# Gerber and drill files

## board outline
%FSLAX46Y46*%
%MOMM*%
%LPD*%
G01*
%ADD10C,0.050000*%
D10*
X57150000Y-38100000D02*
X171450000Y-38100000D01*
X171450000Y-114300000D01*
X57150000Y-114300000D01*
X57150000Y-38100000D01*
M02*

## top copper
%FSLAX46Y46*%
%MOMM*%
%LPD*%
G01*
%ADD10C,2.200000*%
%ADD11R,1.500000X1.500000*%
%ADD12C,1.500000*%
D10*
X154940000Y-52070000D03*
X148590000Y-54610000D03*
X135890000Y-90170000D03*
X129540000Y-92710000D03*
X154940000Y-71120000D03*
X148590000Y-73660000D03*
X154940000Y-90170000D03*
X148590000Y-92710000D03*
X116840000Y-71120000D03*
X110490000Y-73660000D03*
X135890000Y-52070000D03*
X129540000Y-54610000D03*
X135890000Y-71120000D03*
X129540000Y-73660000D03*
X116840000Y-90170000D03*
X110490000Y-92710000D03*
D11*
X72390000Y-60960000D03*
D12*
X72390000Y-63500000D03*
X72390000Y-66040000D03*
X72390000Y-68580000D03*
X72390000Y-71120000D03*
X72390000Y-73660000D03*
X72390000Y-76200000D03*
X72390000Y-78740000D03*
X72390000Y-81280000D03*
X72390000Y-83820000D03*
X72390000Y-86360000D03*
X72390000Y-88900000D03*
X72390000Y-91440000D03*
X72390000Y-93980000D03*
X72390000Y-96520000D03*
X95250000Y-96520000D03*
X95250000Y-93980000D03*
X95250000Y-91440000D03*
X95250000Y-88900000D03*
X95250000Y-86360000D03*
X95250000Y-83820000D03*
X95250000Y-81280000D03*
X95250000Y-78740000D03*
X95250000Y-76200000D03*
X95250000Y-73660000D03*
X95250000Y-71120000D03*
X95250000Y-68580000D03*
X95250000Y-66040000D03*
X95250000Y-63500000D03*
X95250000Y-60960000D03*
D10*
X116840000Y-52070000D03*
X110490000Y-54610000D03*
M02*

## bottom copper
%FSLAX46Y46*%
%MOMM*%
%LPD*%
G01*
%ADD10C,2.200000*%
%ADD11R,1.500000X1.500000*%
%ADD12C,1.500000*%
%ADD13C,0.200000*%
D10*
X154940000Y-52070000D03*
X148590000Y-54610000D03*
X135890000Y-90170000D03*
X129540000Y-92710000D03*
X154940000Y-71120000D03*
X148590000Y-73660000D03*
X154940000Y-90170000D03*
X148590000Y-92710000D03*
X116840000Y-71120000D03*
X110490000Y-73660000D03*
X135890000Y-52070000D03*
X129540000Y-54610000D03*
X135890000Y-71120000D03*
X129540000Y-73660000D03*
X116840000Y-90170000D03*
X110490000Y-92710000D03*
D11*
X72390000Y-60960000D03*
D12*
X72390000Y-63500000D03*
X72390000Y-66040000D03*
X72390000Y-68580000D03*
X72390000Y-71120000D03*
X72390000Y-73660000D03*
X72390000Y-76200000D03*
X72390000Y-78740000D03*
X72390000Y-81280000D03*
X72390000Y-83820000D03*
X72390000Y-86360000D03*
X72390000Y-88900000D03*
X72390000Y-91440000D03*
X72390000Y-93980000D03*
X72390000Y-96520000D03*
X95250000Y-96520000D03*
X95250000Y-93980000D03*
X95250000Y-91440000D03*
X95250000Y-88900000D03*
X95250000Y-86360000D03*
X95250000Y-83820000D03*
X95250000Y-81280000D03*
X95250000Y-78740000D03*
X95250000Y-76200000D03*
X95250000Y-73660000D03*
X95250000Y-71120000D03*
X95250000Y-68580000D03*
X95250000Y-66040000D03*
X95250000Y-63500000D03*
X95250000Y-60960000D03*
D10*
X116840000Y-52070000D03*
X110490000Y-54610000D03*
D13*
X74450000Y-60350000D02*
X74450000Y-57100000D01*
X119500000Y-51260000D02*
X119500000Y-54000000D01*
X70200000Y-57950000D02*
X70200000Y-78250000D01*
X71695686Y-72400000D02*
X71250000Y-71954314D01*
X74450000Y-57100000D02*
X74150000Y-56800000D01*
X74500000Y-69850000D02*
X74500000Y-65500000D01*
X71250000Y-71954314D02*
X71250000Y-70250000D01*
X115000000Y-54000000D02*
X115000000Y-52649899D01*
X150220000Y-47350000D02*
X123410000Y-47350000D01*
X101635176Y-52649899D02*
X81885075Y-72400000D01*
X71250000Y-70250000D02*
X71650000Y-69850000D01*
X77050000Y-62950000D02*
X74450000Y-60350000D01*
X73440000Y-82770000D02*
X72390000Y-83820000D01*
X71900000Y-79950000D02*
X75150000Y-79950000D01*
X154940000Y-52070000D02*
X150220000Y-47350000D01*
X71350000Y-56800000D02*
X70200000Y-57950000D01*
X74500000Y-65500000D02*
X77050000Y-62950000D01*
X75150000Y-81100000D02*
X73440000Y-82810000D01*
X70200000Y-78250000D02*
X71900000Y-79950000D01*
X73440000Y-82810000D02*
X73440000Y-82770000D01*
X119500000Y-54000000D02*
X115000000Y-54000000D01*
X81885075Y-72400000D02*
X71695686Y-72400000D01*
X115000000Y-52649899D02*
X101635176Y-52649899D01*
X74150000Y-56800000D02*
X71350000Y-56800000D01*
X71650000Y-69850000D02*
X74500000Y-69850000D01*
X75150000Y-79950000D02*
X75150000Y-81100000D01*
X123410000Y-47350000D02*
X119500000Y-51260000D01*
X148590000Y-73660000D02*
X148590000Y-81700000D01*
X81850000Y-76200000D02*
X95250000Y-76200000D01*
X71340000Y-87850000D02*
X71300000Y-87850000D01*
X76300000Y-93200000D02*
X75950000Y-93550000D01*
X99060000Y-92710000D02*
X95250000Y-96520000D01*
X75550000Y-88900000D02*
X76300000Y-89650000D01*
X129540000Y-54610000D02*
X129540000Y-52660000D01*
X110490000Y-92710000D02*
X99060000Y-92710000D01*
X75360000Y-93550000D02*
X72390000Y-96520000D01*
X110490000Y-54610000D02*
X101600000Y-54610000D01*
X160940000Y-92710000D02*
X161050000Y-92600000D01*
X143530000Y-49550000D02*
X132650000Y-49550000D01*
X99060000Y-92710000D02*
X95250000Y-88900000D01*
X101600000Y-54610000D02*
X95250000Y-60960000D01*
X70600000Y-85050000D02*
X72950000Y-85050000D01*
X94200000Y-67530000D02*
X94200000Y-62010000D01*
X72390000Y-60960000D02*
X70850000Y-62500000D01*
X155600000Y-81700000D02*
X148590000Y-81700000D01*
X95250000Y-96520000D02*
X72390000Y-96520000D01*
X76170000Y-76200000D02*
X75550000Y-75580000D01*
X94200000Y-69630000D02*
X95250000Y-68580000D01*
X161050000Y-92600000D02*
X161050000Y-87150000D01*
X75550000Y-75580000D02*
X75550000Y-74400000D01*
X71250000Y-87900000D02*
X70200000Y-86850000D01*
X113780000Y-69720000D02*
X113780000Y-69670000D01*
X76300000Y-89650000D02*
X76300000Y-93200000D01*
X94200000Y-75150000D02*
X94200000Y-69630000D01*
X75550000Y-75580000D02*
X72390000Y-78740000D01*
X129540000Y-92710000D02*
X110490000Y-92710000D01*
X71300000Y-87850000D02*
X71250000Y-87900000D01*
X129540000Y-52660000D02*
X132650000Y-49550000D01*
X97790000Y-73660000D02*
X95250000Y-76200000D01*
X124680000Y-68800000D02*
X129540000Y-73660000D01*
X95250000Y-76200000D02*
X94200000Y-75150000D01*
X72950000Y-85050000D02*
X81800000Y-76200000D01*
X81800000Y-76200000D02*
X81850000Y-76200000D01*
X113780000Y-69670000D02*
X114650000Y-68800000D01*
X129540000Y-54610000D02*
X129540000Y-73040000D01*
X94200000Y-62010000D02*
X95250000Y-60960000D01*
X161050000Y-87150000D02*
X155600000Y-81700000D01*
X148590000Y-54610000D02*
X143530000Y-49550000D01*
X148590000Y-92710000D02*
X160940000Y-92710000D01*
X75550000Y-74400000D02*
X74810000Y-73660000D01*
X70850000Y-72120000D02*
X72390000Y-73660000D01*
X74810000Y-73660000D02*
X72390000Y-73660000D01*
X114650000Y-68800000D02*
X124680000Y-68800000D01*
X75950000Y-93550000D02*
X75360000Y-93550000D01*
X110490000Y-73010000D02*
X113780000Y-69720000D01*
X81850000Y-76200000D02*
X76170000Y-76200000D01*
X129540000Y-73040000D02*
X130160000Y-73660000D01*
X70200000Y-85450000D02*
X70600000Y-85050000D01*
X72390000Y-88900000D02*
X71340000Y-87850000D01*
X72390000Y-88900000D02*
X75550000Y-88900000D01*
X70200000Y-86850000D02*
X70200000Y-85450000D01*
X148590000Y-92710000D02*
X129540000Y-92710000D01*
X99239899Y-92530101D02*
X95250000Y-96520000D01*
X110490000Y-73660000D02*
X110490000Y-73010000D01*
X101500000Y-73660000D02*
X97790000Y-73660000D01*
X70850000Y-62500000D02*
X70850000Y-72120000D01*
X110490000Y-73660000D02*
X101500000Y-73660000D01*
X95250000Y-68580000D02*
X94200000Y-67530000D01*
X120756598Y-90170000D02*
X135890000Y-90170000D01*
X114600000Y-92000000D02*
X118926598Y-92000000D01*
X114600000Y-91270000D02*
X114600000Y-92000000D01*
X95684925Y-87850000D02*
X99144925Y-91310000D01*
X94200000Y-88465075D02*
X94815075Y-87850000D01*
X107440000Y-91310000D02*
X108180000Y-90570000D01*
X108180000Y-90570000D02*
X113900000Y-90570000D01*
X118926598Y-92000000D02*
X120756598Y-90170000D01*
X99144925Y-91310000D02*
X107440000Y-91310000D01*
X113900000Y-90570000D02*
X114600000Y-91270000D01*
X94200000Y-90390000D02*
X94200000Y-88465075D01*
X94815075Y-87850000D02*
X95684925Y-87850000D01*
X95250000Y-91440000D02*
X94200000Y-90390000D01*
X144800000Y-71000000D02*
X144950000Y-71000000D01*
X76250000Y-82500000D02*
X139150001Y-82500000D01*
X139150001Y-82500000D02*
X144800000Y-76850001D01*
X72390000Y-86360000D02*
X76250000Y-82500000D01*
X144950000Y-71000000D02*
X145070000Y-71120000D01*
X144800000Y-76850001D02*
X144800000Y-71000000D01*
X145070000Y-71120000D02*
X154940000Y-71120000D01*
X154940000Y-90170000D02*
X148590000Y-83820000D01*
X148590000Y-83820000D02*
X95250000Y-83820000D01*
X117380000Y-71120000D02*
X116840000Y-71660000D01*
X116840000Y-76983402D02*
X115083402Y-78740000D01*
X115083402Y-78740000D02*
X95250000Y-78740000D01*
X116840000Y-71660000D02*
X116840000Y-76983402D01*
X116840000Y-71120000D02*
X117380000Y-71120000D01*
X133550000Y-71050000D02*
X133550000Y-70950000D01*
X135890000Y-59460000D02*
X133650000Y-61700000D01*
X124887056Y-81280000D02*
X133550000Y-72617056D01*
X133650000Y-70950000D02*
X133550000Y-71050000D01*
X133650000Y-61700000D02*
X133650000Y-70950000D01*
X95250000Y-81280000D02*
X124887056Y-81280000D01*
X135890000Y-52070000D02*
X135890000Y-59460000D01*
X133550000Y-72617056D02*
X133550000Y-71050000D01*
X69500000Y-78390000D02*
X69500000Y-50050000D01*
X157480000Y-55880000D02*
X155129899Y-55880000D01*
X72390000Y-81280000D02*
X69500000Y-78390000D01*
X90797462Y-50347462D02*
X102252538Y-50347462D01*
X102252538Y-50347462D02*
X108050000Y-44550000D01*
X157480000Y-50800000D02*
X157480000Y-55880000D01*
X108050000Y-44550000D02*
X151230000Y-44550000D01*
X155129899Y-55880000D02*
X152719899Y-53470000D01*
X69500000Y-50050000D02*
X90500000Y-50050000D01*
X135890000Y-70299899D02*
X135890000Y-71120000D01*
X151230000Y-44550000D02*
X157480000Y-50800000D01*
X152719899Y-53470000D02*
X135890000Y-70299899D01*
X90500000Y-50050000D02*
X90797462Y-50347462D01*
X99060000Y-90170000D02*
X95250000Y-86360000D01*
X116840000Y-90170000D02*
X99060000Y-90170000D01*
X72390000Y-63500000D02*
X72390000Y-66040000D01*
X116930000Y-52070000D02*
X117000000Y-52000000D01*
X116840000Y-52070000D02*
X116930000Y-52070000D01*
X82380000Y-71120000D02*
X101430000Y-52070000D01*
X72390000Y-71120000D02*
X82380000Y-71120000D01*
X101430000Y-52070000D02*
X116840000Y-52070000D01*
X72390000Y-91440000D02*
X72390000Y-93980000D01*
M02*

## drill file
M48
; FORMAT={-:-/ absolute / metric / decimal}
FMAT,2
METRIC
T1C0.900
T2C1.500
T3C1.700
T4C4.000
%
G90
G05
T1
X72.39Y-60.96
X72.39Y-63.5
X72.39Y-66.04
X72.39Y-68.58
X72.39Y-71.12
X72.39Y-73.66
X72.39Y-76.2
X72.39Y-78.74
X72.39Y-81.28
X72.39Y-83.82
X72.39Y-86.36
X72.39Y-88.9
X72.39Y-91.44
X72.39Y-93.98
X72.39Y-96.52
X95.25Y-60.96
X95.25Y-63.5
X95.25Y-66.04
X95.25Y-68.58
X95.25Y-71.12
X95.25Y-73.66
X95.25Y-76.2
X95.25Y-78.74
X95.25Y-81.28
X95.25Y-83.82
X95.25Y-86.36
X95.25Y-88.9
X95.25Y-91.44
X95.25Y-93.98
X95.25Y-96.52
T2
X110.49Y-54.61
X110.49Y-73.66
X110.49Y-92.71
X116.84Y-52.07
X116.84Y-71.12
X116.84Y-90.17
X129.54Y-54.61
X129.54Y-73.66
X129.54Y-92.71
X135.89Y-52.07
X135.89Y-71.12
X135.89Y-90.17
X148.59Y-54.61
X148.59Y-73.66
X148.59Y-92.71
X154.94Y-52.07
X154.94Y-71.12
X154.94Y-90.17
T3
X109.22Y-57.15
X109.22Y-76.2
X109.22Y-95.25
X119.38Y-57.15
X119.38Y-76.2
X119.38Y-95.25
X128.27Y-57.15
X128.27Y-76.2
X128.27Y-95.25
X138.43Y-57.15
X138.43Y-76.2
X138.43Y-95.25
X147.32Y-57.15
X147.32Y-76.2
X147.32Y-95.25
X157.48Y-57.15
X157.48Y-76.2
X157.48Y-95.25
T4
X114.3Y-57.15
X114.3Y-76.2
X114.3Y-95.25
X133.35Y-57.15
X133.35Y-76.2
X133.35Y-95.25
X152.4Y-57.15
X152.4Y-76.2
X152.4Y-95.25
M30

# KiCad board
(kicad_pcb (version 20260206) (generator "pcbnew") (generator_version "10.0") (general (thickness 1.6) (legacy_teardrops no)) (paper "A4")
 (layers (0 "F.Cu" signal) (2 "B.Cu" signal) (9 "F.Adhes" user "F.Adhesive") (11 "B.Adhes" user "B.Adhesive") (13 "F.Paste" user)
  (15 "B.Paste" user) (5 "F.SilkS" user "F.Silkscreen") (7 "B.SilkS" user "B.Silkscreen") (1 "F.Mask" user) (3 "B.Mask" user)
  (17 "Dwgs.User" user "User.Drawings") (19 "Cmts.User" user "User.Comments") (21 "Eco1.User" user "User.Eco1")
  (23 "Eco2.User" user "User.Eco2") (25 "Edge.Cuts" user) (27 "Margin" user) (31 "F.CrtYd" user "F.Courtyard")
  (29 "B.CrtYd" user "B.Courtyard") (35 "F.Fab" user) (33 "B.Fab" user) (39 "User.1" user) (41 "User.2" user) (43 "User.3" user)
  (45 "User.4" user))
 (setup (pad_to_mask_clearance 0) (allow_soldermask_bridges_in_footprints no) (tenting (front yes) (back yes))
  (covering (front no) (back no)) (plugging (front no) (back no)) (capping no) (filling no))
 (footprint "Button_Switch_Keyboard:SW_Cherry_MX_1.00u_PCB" (layer "F.Cu") (at 154.94 52.07)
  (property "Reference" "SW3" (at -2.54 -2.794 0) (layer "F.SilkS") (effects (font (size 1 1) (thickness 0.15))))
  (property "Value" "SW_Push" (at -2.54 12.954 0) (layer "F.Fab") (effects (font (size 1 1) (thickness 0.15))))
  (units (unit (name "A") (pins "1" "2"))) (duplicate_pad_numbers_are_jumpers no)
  (pad "" np_thru_hole circle (at -7.62 5.08) (size 1.7 1.7) (drill 1.7) (layers "*.Cu" "*.Mask"))
  (pad "" np_thru_hole circle (at -2.54 5.08) (size 4 4) (drill 4) (layers "*.Cu" "*.Mask"))
  (pad "" np_thru_hole circle (at 2.54 5.08) (size 1.7 1.7) (drill 1.7) (layers "*.Cu" "*.Mask"))
  (pad "1" thru_hole circle (at 0 0) (size 2.2 2.2) (drill 1.5) (layers "*.Cu" "*.Mask") (remove_unused_layers no) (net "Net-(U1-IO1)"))
  (pad "2" thru_hole circle (at -6.35 2.54) (size 2.2 2.2) (drill 1.5) (layers "*.Cu" "*.Mask") (remove_unused_layers no)
   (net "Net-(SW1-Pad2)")))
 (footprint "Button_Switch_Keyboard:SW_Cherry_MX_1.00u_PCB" (layer "F.Cu") (at 135.89 90.17)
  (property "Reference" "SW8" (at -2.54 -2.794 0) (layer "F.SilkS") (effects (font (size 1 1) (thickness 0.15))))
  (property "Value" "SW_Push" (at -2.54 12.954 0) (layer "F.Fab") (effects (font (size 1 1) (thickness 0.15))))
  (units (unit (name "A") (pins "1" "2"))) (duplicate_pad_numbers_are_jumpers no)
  (pad "" np_thru_hole circle (at -7.62 5.08) (size 1.7 1.7) (drill 1.7) (layers "*.Cu" "*.Mask"))
  (pad "" np_thru_hole circle (at -2.54 5.08) (size 4 4) (drill 4) (layers "*.Cu" "*.Mask"))
  (pad "" np_thru_hole circle (at 2.54 5.08) (size 1.7 1.7) (drill 1.7) (layers "*.Cu" "*.Mask"))
  (pad "1" thru_hole circle (at 0 0) (size 2.2 2.2) (drill 1.5) (layers "*.Cu" "*.Mask") (remove_unused_layers no) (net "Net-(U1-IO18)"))
  (pad "2" thru_hole circle (at -6.35 2.54) (size 2.2 2.2) (drill 1.5) (layers "*.Cu" "*.Mask") (remove_unused_layers no)
   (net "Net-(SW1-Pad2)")))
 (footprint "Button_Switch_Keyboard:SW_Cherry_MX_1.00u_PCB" (layer "F.Cu") (at 154.94 71.12)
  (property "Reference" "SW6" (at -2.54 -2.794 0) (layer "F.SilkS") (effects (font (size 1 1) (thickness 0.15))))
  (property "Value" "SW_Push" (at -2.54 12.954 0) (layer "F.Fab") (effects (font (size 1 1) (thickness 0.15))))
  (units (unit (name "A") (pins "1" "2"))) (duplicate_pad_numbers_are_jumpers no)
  (pad "" np_thru_hole circle (at -7.62 5.08) (size 1.7 1.7) (drill 1.7) (layers "*.Cu" "*.Mask"))
  (pad "" np_thru_hole circle (at -2.54 5.08) (size 4 4) (drill 4) (layers "*.Cu" "*.Mask"))
  (pad "" np_thru_hole circle (at 2.54 5.08) (size 1.7 1.7) (drill 1.7) (layers "*.Cu" "*.Mask"))
  (pad "1" thru_hole circle (at 0 0) (size 2.2 2.2) (drill 1.5) (layers "*.Cu" "*.Mask") (remove_unused_layers no) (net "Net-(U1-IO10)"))
  (pad "2" thru_hole circle (at -6.35 2.54) (size 2.2 2.2) (drill 1.5) (layers "*.Cu" "*.Mask") (remove_unused_layers no)
   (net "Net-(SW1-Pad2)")))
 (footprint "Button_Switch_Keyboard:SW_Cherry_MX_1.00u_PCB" (layer "F.Cu") (at 154.94 90.17)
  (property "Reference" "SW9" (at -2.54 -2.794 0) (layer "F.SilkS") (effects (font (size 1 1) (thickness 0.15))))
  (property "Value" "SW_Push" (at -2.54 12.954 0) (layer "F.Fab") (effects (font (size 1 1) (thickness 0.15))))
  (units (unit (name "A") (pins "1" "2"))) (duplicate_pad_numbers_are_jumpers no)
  (pad "" np_thru_hole circle (at -7.62 5.08) (size 1.7 1.7) (drill 1.7) (layers "*.Cu" "*.Mask"))
  (pad "" np_thru_hole circle (at -2.54 5.08) (size 4 4) (drill 4) (layers "*.Cu" "*.Mask"))
  (pad "" np_thru_hole circle (at 2.54 5.08) (size 1.7 1.7) (drill 1.7) (layers "*.Cu" "*.Mask"))
  (pad "1" thru_hole circle (at 0 0) (size 2.2 2.2) (drill 1.5) (layers "*.Cu" "*.Mask") (remove_unused_layers no) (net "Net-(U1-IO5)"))
  (pad "2" thru_hole circle (at -6.35 2.54) (size 2.2 2.2) (drill 1.5) (layers "*.Cu" "*.Mask") (remove_unused_layers no)
   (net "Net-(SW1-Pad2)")))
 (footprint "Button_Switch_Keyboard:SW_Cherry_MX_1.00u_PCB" (layer "F.Cu") (at 116.84 71.12)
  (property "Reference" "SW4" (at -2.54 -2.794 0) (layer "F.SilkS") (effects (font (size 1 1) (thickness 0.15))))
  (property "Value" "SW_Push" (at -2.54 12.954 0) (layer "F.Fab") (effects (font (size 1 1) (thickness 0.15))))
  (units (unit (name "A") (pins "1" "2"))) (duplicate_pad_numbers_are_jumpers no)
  (pad "" np_thru_hole circle (at -7.62 5.08) (size 1.7 1.7) (drill 1.7) (layers "*.Cu" "*.Mask"))
  (pad "" np_thru_hole circle (at -2.54 5.08) (size 4 4) (drill 4) (layers "*.Cu" "*.Mask"))
  (pad "" np_thru_hole circle (at 2.54 5.08) (size 1.7 1.7) (drill 1.7) (layers "*.Cu" "*.Mask"))
  (pad "1" thru_hole circle (at 0 0) (size 2.2 2.2) (drill 1.5) (layers "*.Cu" "*.Mask") (remove_unused_layers no) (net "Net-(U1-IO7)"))
  (pad "2" thru_hole circle (at -6.35 2.54) (size 2.2 2.2) (drill 1.5) (layers "*.Cu" "*.Mask") (remove_unused_layers no)
   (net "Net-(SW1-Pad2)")))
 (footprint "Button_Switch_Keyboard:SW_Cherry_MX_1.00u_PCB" (layer "F.Cu") (at 135.89 52.07)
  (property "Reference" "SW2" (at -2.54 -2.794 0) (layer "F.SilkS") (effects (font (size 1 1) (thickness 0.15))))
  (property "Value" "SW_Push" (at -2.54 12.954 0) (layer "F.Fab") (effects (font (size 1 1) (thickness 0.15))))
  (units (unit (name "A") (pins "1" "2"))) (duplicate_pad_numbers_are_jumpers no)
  (pad "" np_thru_hole circle (at -7.62 5.08) (size 1.7 1.7) (drill 1.7) (layers "*.Cu" "*.Mask"))
  (pad "" np_thru_hole circle (at -2.54 5.08) (size 4 4) (drill 4) (layers "*.Cu" "*.Mask"))
  (pad "" np_thru_hole circle (at 2.54 5.08) (size 1.7 1.7) (drill 1.7) (layers "*.Cu" "*.Mask"))
  (pad "1" thru_hole circle (at 0 0) (size 2.2 2.2) (drill 1.5) (layers "*.Cu" "*.Mask") (remove_unused_layers no) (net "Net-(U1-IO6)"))
  (pad "2" thru_hole circle (at -6.35 2.54) (size 2.2 2.2) (drill 1.5) (layers "*.Cu" "*.Mask") (remove_unused_layers no)
   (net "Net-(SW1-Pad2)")))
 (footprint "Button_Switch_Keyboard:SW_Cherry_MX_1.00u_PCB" (layer "F.Cu") (at 135.89 71.12)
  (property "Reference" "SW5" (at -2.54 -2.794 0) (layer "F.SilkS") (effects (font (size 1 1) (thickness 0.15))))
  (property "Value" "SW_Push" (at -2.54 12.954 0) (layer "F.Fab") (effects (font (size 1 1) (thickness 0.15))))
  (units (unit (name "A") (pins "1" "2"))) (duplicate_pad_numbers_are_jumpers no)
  (pad "" np_thru_hole circle (at -7.62 5.08) (size 1.7 1.7) (drill 1.7) (layers "*.Cu" "*.Mask"))
  (pad "" np_thru_hole circle (at -2.54 5.08) (size 4 4) (drill 4) (layers "*.Cu" "*.Mask"))
  (pad "" np_thru_hole circle (at 2.54 5.08) (size 1.7 1.7) (drill 1.7) (layers "*.Cu" "*.Mask"))
  (pad "1" thru_hole circle (at 0 0) (size 2.2 2.2) (drill 1.5) (layers "*.Cu" "*.Mask") (remove_unused_layers no) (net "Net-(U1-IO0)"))
  (pad "2" thru_hole circle (at -6.35 2.54) (size 2.2 2.2) (drill 1.5) (layers "*.Cu" "*.Mask") (remove_unused_layers no)
   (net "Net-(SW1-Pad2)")))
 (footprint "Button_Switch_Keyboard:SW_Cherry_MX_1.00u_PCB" (layer "F.Cu") (at 116.84 90.17)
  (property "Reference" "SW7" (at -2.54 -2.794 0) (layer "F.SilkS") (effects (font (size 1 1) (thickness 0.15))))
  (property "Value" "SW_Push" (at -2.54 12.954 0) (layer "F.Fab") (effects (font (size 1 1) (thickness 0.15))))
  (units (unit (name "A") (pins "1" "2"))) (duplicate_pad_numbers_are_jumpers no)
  (pad "" np_thru_hole circle (at -7.62 5.08) (size 1.7 1.7) (drill 1.7) (layers "*.Cu" "*.Mask"))
  (pad "" np_thru_hole circle (at -2.54 5.08) (size 4 4) (drill 4) (layers "*.Cu" "*.Mask"))
  (pad "" np_thru_hole circle (at 2.54 5.08) (size 1.7 1.7) (drill 1.7) (layers "*.Cu" "*.Mask"))
  (pad "1" thru_hole circle (at 0 0) (size 2.2 2.2) (drill 1.5) (layers "*.Cu" "*.Mask") (remove_unused_layers no) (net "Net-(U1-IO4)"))
  (pad "2" thru_hole circle (at -6.35 2.54) (size 2.2 2.2) (drill 1.5) (layers "*.Cu" "*.Mask") (remove_unused_layers no)
   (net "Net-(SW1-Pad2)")))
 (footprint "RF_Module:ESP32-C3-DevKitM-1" (layer "F.Cu") (at 72.39 60.96)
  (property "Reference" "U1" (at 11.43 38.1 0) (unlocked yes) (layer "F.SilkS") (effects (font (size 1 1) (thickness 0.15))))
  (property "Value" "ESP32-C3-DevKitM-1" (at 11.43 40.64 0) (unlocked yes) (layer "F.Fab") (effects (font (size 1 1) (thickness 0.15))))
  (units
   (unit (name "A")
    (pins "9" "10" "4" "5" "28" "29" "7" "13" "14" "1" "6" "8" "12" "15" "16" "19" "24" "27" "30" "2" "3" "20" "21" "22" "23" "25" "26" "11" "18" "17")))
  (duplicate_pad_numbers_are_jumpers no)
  (pad "1" thru_hole rect (at 0 0) (size 1.5 1.5) (drill 0.9) (layers "*.Cu" "*.Mask") (remove_unused_layers yes) (keep_end_layers yes)
   (zone_layer_connections) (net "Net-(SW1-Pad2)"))
  (pad "2" thru_hole circle (at 0 2.54) (size 1.5 1.5) (drill 0.9) (layers "*.Cu" "*.Mask") (remove_unused_layers yes) (keep_end_layers yes)
   (zone_layer_connections) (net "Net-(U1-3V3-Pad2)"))
  (pad "3" thru_hole circle (at 0 5.08) (size 1.5 1.5) (drill 0.9) (layers "*.Cu" "*.Mask") (remove_unused_layers yes) (keep_end_layers yes)
   (zone_layer_connections) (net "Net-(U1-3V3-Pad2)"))
  (pad "4" thru_hole circle (at 0 7.62) (size 1.5 1.5) (drill 0.9) (layers "*.Cu" "*.Mask") (remove_unused_layers yes) (keep_end_layers yes)
   (zone_layer_connections) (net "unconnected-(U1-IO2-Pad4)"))
  (pad "5" thru_hole circle (at 0 10.16) (size 1.5 1.5) (drill 0.9) (layers "*.Cu" "*.Mask") (remove_unused_layers yes)
   (keep_end_layers yes) (zone_layer_connections) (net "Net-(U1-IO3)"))
  (pad "6" thru_hole circle (at 0 12.7) (size 1.5 1.5) (drill 0.9) (layers "*.Cu" "*.Mask") (remove_unused_layers yes) (keep_end_layers yes)
   (zone_layer_connections) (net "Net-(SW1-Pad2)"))
  (pad "7" thru_hole circle (at 0 15.24) (size 1.5 1.5) (drill 0.9) (layers "*.Cu" "*.Mask") (remove_unused_layers yes)
   (keep_end_layers yes) (zone_layer_connections) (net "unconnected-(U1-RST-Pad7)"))
  (pad "8" thru_hole circle (at 0 17.78) (size 1.5 1.5) (drill 0.9) (layers "*.Cu" "*.Mask") (remove_unused_layers yes)
   (keep_end_layers yes) (zone_layer_connections) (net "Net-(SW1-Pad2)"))
  (pad "9" thru_hole circle (at 0 20.32) (size 1.5 1.5) (drill 0.9) (layers "*.Cu" "*.Mask") (remove_unused_layers yes)
   (keep_end_layers yes) (zone_layer_connections) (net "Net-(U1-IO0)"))
  (pad "10" thru_hole circle (at 0 22.86) (size 1.5 1.5) (drill 0.9) (layers "*.Cu" "*.Mask") (remove_unused_layers yes)
   (keep_end_layers yes) (zone_layer_connections) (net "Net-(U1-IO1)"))
  (pad "11" thru_hole circle (at 0 25.4) (size 1.5 1.5) (drill 0.9) (layers "*.Cu" "*.Mask") (remove_unused_layers yes)
   (keep_end_layers yes) (zone_layer_connections) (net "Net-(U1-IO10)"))
  (pad "12" thru_hole circle (at 0 27.94) (size 1.5 1.5) (drill 0.9) (layers "*.Cu" "*.Mask") (remove_unused_layers yes)
   (keep_end_layers yes) (zone_layer_connections) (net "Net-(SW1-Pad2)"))
  (pad "13" thru_hole circle (at 0 30.48) (size 1.5 1.5) (drill 0.9) (layers "*.Cu" "*.Mask") (remove_unused_layers yes)
   (keep_end_layers yes) (zone_layer_connections) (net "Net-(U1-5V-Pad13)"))
  (pad "14" thru_hole circle (at 0 33.02) (size 1.5 1.5) (drill 0.9) (layers "*.Cu" "*.Mask") (remove_unused_layers yes)
   (keep_end_layers yes) (zone_layer_connections) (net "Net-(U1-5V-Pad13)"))
  (pad "15" thru_hole circle (at 0 35.56) (size 1.5 1.5) (drill 0.9) (layers "*.Cu" "*.Mask") (remove_unused_layers yes)
   (keep_end_layers yes) (zone_layer_connections) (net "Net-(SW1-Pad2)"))
  (pad "16" thru_hole circle (at 22.86 35.56) (size 1.5 1.5) (drill 0.9) (layers "*.Cu" "*.Mask") (remove_unused_layers yes)
   (keep_end_layers yes) (zone_layer_connections) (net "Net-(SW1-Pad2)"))
  (pad "17" thru_hole circle (at 22.86 33.02) (size 1.5 1.5) (drill 0.9) (layers "*.Cu" "*.Mask") (remove_unused_layers yes)
   (keep_end_layers yes) (zone_layer_connections) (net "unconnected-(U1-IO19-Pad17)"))
  (pad "18" thru_hole circle (at 22.86 30.48) (size 1.5 1.5) (drill 0.9) (layers "*.Cu" "*.Mask") (remove_unused_layers yes)
   (keep_end_layers yes) (zone_layer_connections) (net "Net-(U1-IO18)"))
  (pad "19" thru_hole circle (at 22.86 27.94) (size 1.5 1.5) (drill 0.9) (layers "*.Cu" "*.Mask") (remove_unused_layers yes)
   (keep_end_layers yes) (zone_layer_connections) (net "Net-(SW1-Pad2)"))
  (pad "20" thru_hole circle (at 22.86 25.4) (size 1.5 1.5) (drill 0.9) (layers "*.Cu" "*.Mask") (remove_unused_layers yes)
   (keep_end_layers yes) (zone_layer_connections) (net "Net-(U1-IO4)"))
  (pad "21" thru_hole circle (at 22.86 22.86) (size 1.5 1.5) (drill 0.9) (layers "*.Cu" "*.Mask") (remove_unused_layers yes)
   (keep_end_layers yes) (zone_layer_connections) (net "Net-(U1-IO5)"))
  (pad "22" thru_hole circle (at 22.86 20.32) (size 1.5 1.5) (drill 0.9) (layers "*.Cu" "*.Mask") (remove_unused_layers yes)
   (keep_end_layers yes) (zone_layer_connections) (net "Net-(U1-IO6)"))
  (pad "23" thru_hole circle (at 22.86 17.78) (size 1.5 1.5) (drill 0.9) (layers "*.Cu" "*.Mask") (remove_unused_layers yes)
   (keep_end_layers yes) (zone_layer_connections) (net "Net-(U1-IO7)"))
  (pad "24" thru_hole circle (at 22.86 15.24) (size 1.5 1.5) (drill 0.9) (layers "*.Cu" "*.Mask") (remove_unused_layers yes)
   (keep_end_layers yes) (zone_layer_connections) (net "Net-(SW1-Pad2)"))
  (pad "25" thru_hole circle (at 22.86 12.7) (size 1.5 1.5) (drill 0.9) (layers "*.Cu" "*.Mask") (remove_unused_layers yes)
   (keep_end_layers yes) (zone_layer_connections) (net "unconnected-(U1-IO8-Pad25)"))
  (pad "26" thru_hole circle (at 22.86 10.16) (size 1.5 1.5) (drill 0.9) (layers "*.Cu" "*.Mask") (remove_unused_layers yes)
   (keep_end_layers yes) (zone_layer_connections) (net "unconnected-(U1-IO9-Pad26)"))
  (pad "27" thru_hole circle (at 22.86 7.62) (size 1.5 1.5) (drill 0.9) (layers "*.Cu" "*.Mask") (remove_unused_layers yes)
   (keep_end_layers yes) (zone_layer_connections) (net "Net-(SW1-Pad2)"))
  (pad "28" thru_hole circle (at 22.86 5.08) (size 1.5 1.5) (drill 0.9) (layers "*.Cu" "*.Mask") (remove_unused_layers yes)
   (keep_end_layers yes) (zone_layer_connections) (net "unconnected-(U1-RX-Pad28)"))
  (pad "29" thru_hole circle (at 22.86 2.54) (size 1.5 1.5) (drill 0.9) (layers "*.Cu" "*.Mask") (remove_unused_layers yes)
   (keep_end_layers yes) (zone_layer_connections) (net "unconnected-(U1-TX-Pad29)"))
  (pad "30" thru_hole circle (at 22.86 0) (size 1.5 1.5) (drill 0.9) (layers "*.Cu" "*.Mask") (remove_unused_layers yes)
   (keep_end_layers yes) (zone_layer_connections) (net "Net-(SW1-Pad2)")))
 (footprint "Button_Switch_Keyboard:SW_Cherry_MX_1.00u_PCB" (layer "F.Cu") (at 116.84 52.07)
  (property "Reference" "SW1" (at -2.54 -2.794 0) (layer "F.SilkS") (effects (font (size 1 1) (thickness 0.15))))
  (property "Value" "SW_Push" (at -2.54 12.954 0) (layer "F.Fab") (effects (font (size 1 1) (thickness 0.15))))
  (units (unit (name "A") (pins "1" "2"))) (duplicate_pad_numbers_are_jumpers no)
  (pad "" np_thru_hole circle (at -7.62 5.08) (size 1.7 1.7) (drill 1.7) (layers "*.Cu" "*.Mask"))
  (pad "" np_thru_hole circle (at -2.54 5.08) (size 4 4) (drill 4) (layers "*.Cu" "*.Mask"))
  (pad "" np_thru_hole circle (at 2.54 5.08) (size 1.7 1.7) (drill 1.7) (layers "*.Cu" "*.Mask"))
  (pad "1" thru_hole circle (at 0 0) (size 2.2 2.2) (drill 1.5) (layers "*.Cu" "*.Mask") (remove_unused_layers no) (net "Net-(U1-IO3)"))
  (pad "2" thru_hole circle (at -6.35 2.54) (size 2.2 2.2) (drill 1.5) (layers "*.Cu" "*.Mask") (remove_unused_layers no)
   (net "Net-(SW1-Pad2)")))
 (gr_rect (start 57.15 38.1) (end 171.45 114.3) (stroke (width 0.05) (type default)) (fill no) (layer "Edge.Cuts"))
 (segment (start 74.45 60.35) (end 74.45 57.1) (width 0.2) (layer "B.Cu") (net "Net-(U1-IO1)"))
 (segment (start 119.5 51.26) (end 119.5 54) (width 0.2) (layer "B.Cu") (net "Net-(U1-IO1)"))
 (segment (start 70.2 57.95) (end 70.2 78.25) (width 0.2) (layer "B.Cu") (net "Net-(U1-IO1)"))
 (segment (start 71.695686 72.4) (end 71.25 71.954314) (width 0.2) (layer "B.Cu") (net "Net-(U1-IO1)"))
 (segment (start 74.45 57.1) (end 74.15 56.8) (width 0.2) (layer "B.Cu") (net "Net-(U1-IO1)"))
 (segment (start 74.5 69.85) (end 74.5 65.5) (width 0.2) (layer "B.Cu") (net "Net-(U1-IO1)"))
 (segment (start 71.25 71.954314) (end 71.25 70.25) (width 0.2) (layer "B.Cu") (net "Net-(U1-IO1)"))
 (segment (start 115 54) (end 115 52.649899) (width 0.2) (layer "B.Cu") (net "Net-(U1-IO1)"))
 (segment (start 150.22 47.35) (end 123.41 47.35) (width 0.2) (layer "B.Cu") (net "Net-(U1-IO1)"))
 (segment (start 101.635176 52.649899) (end 81.885075 72.4) (width 0.2) (layer "B.Cu") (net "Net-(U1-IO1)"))
 (segment (start 71.25 70.25) (end 71.65 69.85) (width 0.2) (layer "B.Cu") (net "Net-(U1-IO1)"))
 (segment (start 77.05 62.95) (end 74.45 60.35) (width 0.2) (layer "B.Cu") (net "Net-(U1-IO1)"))
 (segment (start 73.44 82.77) (end 72.39 83.82) (width 0.2) (layer "B.Cu") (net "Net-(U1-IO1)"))
 (segment (start 71.9 79.95) (end 75.15 79.95) (width 0.2) (layer "B.Cu") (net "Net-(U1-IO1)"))
 (segment (start 154.94 52.07) (end 150.22 47.35) (width 0.2) (layer "B.Cu") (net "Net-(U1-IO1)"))
 (segment (start 71.35 56.8) (end 70.2 57.95) (width 0.2) (layer "B.Cu") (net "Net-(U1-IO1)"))
 (segment (start 74.5 65.5) (end 77.05 62.95) (width 0.2) (layer "B.Cu") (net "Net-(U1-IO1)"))
 (segment (start 75.15 81.1) (end 73.44 82.81) (width 0.2) (layer "B.Cu") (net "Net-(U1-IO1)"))
 (segment (start 70.2 78.25) (end 71.9 79.95) (width 0.2) (layer "B.Cu") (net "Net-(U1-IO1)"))
 (segment (start 73.44 82.81) (end 73.44 82.77) (width 0.2) (layer "B.Cu") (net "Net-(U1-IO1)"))
 (segment (start 119.5 54) (end 115 54) (width 0.2) (layer "B.Cu") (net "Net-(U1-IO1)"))
 (segment (start 81.885075 72.4) (end 71.695686 72.4) (width 0.2) (layer "B.Cu") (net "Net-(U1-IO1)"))
 (segment (start 115 52.649899) (end 101.635176 52.649899) (width 0.2) (layer "B.Cu") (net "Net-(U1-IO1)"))
 (segment (start 74.15 56.8) (end 71.35 56.8) (width 0.2) (layer "B.Cu") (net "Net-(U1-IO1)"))
 (segment (start 71.65 69.85) (end 74.5 69.85) (width 0.2) (layer "B.Cu") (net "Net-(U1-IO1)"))
 (segment (start 75.15 79.95) (end 75.15 81.1) (width 0.2) (layer "B.Cu") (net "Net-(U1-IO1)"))
 (segment (start 123.41 47.35) (end 119.5 51.26) (width 0.2) (layer "B.Cu") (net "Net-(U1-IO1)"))
 (segment (start 148.59 73.66) (end 148.59 81.7) (width 0.2) (layer "B.Cu") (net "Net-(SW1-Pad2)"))
 (segment (start 81.85 76.2) (end 95.25 76.2) (width 0.2) (layer "B.Cu") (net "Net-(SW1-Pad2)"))
 (segment (start 71.34 87.85) (end 71.3 87.85) (width 0.2) (layer "B.Cu") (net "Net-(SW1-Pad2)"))
 (segment (start 76.3 93.2) (end 75.95 93.55) (width 0.2) (layer "B.Cu") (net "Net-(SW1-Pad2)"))
 (segment (start 99.06 92.71) (end 95.25 96.52) (width 0.2) (layer "B.Cu") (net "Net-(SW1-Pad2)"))
 (segment (start 75.55 88.9) (end 76.3 89.65) (width 0.2) (layer "B.Cu") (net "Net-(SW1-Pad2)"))
 (segment (start 129.54 54.61) (end 129.54 52.66) (width 0.2) (layer "B.Cu") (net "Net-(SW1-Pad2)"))
 (segment (start 110.49 92.71) (end 99.06 92.71) (width 0.2) (layer "B.Cu") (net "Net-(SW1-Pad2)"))
 (segment (start 75.36 93.55) (end 72.39 96.52) (width 0.2) (layer "B.Cu") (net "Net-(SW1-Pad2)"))
 (segment (start 110.49 54.61) (end 101.6 54.61) (width 0.2) (layer "B.Cu") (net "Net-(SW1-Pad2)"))
 (segment (start 160.94 92.71) (end 161.05 92.6) (width 0.2) (layer "B.Cu") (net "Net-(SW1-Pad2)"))
 (segment (start 143.53 49.55) (end 132.65 49.55) (width 0.2) (layer "B.Cu") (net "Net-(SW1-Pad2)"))
 (segment (start 99.06 92.71) (end 95.25 88.9) (width 0.2) (layer "B.Cu") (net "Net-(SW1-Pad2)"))
 (segment (start 101.6 54.61) (end 95.25 60.96) (width 0.2) (layer "B.Cu") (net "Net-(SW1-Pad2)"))
 (segment (start 70.6 85.05) (end 72.95 85.05) (width 0.2) (layer "B.Cu") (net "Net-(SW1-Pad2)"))
 (segment (start 94.2 67.53) (end 94.2 62.01) (width 0.2) (layer "B.Cu") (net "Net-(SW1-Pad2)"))
 (segment (start 72.39 60.96) (end 70.85 62.5) (width 0.2) (layer "B.Cu") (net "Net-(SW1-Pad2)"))
 (segment (start 155.6 81.7) (end 148.59 81.7) (width 0.2) (layer "B.Cu") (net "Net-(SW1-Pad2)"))
 (segment (start 95.25 96.52) (end 72.39 96.52) (width 0.2) (layer "B.Cu") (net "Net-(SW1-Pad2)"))
 (segment (start 76.17 76.2) (end 75.55 75.58) (width 0.2) (layer "B.Cu") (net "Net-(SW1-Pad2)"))
 (segment (start 94.2 69.63) (end 95.25 68.58) (width 0.2) (layer "B.Cu") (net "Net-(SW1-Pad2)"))
 (segment (start 161.05 92.6) (end 161.05 87.15) (width 0.2) (layer "B.Cu") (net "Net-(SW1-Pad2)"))
 (segment (start 75.55 75.58) (end 75.55 74.4) (width 0.2) (layer "B.Cu") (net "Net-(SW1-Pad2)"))
 (segment (start 71.25 87.9) (end 70.2 86.85) (width 0.2) (layer "B.Cu") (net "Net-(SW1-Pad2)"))
 (segment (start 113.78 69.72) (end 113.78 69.67) (width 0.2) (layer "B.Cu") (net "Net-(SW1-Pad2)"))
 (segment (start 76.3 89.65) (end 76.3 93.2) (width 0.2) (layer "B.Cu") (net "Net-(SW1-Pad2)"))
 (segment (start 94.2 75.15) (end 94.2 69.63) (width 0.2) (layer "B.Cu") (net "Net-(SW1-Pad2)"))
 (segment (start 75.55 75.58) (end 72.39 78.74) (width 0.2) (layer "B.Cu") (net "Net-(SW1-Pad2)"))
 (segment (start 129.54 92.71) (end 110.49 92.71) (width 0.2) (layer "B.Cu") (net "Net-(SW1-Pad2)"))
 (segment (start 71.3 87.85) (end 71.25 87.9) (width 0.2) (layer "B.Cu") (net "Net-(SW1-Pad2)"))
 (segment (start 129.54 52.66) (end 132.65 49.55) (width 0.2) (layer "B.Cu") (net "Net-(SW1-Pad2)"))
 (segment (start 97.79 73.66) (end 95.25 76.2) (width 0.2) (layer "B.Cu") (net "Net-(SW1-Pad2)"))
 (segment (start 124.68 68.8) (end 129.54 73.66) (width 0.2) (layer "B.Cu") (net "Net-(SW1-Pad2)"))
 (segment (start 95.25 76.2) (end 94.2 75.15) (width 0.2) (layer "B.Cu") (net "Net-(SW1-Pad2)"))
 (segment (start 72.95 85.05) (end 81.8 76.2) (width 0.2) (layer "B.Cu") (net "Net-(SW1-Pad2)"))
 (segment (start 81.8 76.2) (end 81.85 76.2) (width 0.2) (layer "B.Cu") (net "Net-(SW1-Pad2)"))
 (segment (start 113.78 69.67) (end 114.65 68.8) (width 0.2) (layer "B.Cu") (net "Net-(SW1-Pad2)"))
 (segment (start 129.54 54.61) (end 129.54 73.04) (width 0.2) (layer "B.Cu") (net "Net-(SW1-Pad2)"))
 (segment (start 94.2 62.01) (end 95.25 60.96) (width 0.2) (layer "B.Cu") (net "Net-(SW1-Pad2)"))
 (segment (start 161.05 87.15) (end 155.6 81.7) (width 0.2) (layer "B.Cu") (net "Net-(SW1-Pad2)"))
 (segment (start 148.59 54.61) (end 143.53 49.55) (width 0.2) (layer "B.Cu") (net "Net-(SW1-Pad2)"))
 (segment (start 148.59 92.71) (end 160.94 92.71) (width 0.2) (layer "B.Cu") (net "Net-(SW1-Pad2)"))
 (segment (start 75.55 74.4) (end 74.81 73.66) (width 0.2) (layer "B.Cu") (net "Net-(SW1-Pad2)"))
 (segment (start 70.85 72.12) (end 72.39 73.66) (width 0.2) (layer "B.Cu") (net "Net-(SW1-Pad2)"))
 (segment (start 74.81 73.66) (end 72.39 73.66) (width 0.2) (layer "B.Cu") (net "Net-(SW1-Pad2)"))
 (segment (start 114.65 68.8) (end 124.68 68.8) (width 0.2) (layer "B.Cu") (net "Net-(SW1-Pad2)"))
 (segment (start 75.95 93.55) (end 75.36 93.55) (width 0.2) (layer "B.Cu") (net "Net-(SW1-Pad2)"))
 (segment (start 110.49 73.01) (end 113.78 69.72) (width 0.2) (layer "B.Cu") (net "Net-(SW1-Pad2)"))
 (segment (start 81.85 76.2) (end 76.17 76.2) (width 0.2) (layer "B.Cu") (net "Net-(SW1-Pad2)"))
 (segment (start 129.54 73.04) (end 130.16 73.66) (width 0.2) (layer "B.Cu") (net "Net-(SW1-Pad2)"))
 (segment (start 70.2 85.45) (end 70.6 85.05) (width 0.2) (layer "B.Cu") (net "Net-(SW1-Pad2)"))
 (segment (start 72.39 88.9) (end 71.34 87.85) (width 0.2) (layer "B.Cu") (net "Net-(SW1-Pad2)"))
 (segment (start 72.39 88.9) (end 75.55 88.9) (width 0.2) (layer "B.Cu") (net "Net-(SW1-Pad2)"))
 (segment (start 70.2 86.85) (end 70.2 85.45) (width 0.2) (layer "B.Cu") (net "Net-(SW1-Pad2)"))
 (segment (start 148.59 92.71) (end 129.54 92.71) (width 0.2) (layer "B.Cu") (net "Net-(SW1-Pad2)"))
 (segment (start 99.239899 92.530101) (end 95.25 96.52) (width 0.2) (layer "B.Cu") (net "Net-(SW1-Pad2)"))
 (segment (start 110.49 73.66) (end 110.49 73.01) (width 0.2) (layer "B.Cu") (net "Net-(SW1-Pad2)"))
 (segment (start 101.5 73.66) (end 97.79 73.66) (width 0.2) (layer "B.Cu") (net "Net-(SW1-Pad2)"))
 (segment (start 70.85 62.5) (end 70.85 72.12) (width 0.2) (layer "B.Cu") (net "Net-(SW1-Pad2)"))
 (segment (start 110.49 73.66) (end 101.5 73.66) (width 0.2) (layer "B.Cu") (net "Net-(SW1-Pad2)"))
 (segment (start 95.25 68.58) (end 94.2 67.53) (width 0.2) (layer "B.Cu") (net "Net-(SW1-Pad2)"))
 (segment (start 120.756598 90.17) (end 135.89 90.17) (width 0.2) (layer "B.Cu") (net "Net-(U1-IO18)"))
 (segment (start 114.6 92) (end 118.926598 92) (width 0.2) (layer "B.Cu") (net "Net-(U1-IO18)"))
 (segment (start 114.6 91.27) (end 114.6 92) (width 0.2) (layer "B.Cu") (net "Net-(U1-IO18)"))
 (segment (start 95.684925 87.85) (end 99.144925 91.31) (width 0.2) (layer "B.Cu") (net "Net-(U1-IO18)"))
 (segment (start 94.2 88.465075) (end 94.815075 87.85) (width 0.2) (layer "B.Cu") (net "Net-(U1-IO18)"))
 (segment (start 107.44 91.31) (end 108.18 90.57) (width 0.2) (layer "B.Cu") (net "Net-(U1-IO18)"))
 (segment (start 108.18 90.57) (end 113.9 90.57) (width 0.2) (layer "B.Cu") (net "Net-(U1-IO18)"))
 (segment (start 118.926598 92) (end 120.756598 90.17) (width 0.2) (layer "B.Cu") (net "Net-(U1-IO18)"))
 (segment (start 99.144925 91.31) (end 107.44 91.31) (width 0.2) (layer "B.Cu") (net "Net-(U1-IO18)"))
 (segment (start 113.9 90.57) (end 114.6 91.27) (width 0.2) (layer "B.Cu") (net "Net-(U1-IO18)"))
 (segment (start 94.2 90.39) (end 94.2 88.465075) (width 0.2) (layer "B.Cu") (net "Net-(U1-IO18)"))
 (segment (start 94.815075 87.85) (end 95.684925 87.85) (width 0.2) (layer "B.Cu") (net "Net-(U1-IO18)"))
 (segment (start 95.25 91.44) (end 94.2 90.39) (width 0.2) (layer "B.Cu") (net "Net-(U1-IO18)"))
 (segment (start 144.8 71) (end 144.95 71) (width 0.2) (layer "B.Cu") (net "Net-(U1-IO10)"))
 (segment (start 76.25 82.5) (end 139.150001 82.5) (width 0.2) (layer "B.Cu") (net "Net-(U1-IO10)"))
 (segment (start 139.150001 82.5) (end 144.8 76.850001) (width 0.2) (layer "B.Cu") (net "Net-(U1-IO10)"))
 (segment (start 72.39 86.36) (end 76.25 82.5) (width 0.2) (layer "B.Cu") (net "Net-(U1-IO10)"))
 (segment (start 144.95 71) (end 145.07 71.12) (width 0.2) (layer "B.Cu") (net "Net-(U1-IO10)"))
 (segment (start 144.8 76.850001) (end 144.8 71) (width 0.2) (layer "B.Cu") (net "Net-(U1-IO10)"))
 (segment (start 145.07 71.12) (end 154.94 71.12) (width 0.2) (layer "B.Cu") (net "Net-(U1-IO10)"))
 (segment (start 154.94 90.17) (end 148.59 83.82) (width 0.2) (layer "B.Cu") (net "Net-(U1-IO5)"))
 (segment (start 148.59 83.82) (end 95.25 83.82) (width 0.2) (layer "B.Cu") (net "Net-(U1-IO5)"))
 (segment (start 117.38 71.12) (end 116.84 71.66) (width 0.2) (layer "B.Cu") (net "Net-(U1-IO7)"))
 (segment (start 116.84 76.983402) (end 115.083402 78.74) (width 0.2) (layer "B.Cu") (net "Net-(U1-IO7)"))
 (segment (start 115.083402 78.74) (end 95.25 78.74) (width 0.2) (layer "B.Cu") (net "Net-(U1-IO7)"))
 (segment (start 116.84 71.66) (end 116.84 76.983402) (width 0.2) (layer "B.Cu") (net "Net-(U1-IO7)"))
 (segment (start 116.84 71.12) (end 117.38 71.12) (width 0.2) (layer "B.Cu") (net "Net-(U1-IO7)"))
 (segment (start 133.55 71.05) (end 133.55 70.95) (width 0.2) (layer "B.Cu") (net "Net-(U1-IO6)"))
 (segment (start 135.89 59.46) (end 133.65 61.7) (width 0.2) (layer "B.Cu") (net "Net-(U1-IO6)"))
 (segment (start 124.887056 81.28) (end 133.55 72.617056) (width 0.2) (layer "B.Cu") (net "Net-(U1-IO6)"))
 (segment (start 133.65 70.95) (end 133.55 71.05) (width 0.2) (layer "B.Cu") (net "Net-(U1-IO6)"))
 (segment (start 133.65 61.7) (end 133.65 70.95) (width 0.2) (layer "B.Cu") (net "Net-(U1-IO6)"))
 (segment (start 95.25 81.28) (end 124.887056 81.28) (width 0.2) (layer "B.Cu") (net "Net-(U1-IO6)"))
 (segment (start 135.89 52.07) (end 135.89 59.46) (width 0.2) (layer "B.Cu") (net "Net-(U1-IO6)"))
 (segment (start 133.55 72.617056) (end 133.55 71.05) (width 0.2) (layer "B.Cu") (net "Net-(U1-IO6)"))
 (segment (start 69.5 78.39) (end 69.5 50.05) (width 0.2) (layer "B.Cu") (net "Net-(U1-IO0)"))
 (segment (start 157.48 55.88) (end 155.129899 55.88) (width 0.2) (layer "B.Cu") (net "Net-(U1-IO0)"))
 (segment (start 72.39 81.28) (end 69.5 78.39) (width 0.2) (layer "B.Cu") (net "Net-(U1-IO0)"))
 (segment (start 90.797462 50.347462) (end 102.252538 50.347462) (width 0.2) (layer "B.Cu") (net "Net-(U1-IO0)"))
 (segment (start 102.252538 50.347462) (end 108.05 44.55) (width 0.2) (layer "B.Cu") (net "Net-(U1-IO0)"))
 (segment (start 157.48 50.8) (end 157.48 55.88) (width 0.2) (layer "B.Cu") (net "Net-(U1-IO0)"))
 (segment (start 108.05 44.55) (end 151.23 44.55) (width 0.2) (layer "B.Cu") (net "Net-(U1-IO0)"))
 (segment (start 155.129899 55.88) (end 152.719899 53.47) (width 0.2) (layer "B.Cu") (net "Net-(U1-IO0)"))
 (segment (start 69.5 50.05) (end 90.5 50.05) (width 0.2) (layer "B.Cu") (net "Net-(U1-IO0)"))
 (segment (start 135.89 70.299899) (end 135.89 71.12) (width 0.2) (layer "B.Cu") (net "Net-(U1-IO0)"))
 (segment (start 151.23 44.55) (end 157.48 50.8) (width 0.2) (layer "B.Cu") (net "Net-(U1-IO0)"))
 (segment (start 152.719899 53.47) (end 135.89 70.299899) (width 0.2) (layer "B.Cu") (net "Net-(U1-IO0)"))
 (segment (start 90.5 50.05) (end 90.797462 50.347462) (width 0.2) (layer "B.Cu") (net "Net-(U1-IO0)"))
 (segment (start 99.06 90.17) (end 95.25 86.36) (width 0.2) (layer "B.Cu") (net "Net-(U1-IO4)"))
 (segment (start 116.84 90.17) (end 99.06 90.17) (width 0.2) (layer "B.Cu") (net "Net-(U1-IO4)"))
 (segment (start 72.39 63.5) (end 72.39 66.04) (width 0.2) (layer "B.Cu") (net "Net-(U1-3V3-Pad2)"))
 (segment (start 116.93 52.07) (end 117 52) (width 0.2) (layer "B.Cu") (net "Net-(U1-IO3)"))
 (segment (start 116.84 52.07) (end 116.93 52.07) (width 0.2) (layer "B.Cu") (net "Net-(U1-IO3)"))
 (segment (start 82.38 71.12) (end 101.43 52.07) (width 0.2) (layer "B.Cu") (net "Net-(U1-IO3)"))
 (segment (start 72.39 71.12) (end 82.38 71.12) (width 0.2) (layer "B.Cu") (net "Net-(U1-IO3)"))
 (segment (start 101.43 52.07) (end 116.84 52.07) (width 0.2) (layer "B.Cu") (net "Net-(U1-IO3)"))
 (segment (start 72.39 91.44) (end 72.39 93.98) (width 0.2) (layer "B.Cu") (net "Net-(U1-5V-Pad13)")))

